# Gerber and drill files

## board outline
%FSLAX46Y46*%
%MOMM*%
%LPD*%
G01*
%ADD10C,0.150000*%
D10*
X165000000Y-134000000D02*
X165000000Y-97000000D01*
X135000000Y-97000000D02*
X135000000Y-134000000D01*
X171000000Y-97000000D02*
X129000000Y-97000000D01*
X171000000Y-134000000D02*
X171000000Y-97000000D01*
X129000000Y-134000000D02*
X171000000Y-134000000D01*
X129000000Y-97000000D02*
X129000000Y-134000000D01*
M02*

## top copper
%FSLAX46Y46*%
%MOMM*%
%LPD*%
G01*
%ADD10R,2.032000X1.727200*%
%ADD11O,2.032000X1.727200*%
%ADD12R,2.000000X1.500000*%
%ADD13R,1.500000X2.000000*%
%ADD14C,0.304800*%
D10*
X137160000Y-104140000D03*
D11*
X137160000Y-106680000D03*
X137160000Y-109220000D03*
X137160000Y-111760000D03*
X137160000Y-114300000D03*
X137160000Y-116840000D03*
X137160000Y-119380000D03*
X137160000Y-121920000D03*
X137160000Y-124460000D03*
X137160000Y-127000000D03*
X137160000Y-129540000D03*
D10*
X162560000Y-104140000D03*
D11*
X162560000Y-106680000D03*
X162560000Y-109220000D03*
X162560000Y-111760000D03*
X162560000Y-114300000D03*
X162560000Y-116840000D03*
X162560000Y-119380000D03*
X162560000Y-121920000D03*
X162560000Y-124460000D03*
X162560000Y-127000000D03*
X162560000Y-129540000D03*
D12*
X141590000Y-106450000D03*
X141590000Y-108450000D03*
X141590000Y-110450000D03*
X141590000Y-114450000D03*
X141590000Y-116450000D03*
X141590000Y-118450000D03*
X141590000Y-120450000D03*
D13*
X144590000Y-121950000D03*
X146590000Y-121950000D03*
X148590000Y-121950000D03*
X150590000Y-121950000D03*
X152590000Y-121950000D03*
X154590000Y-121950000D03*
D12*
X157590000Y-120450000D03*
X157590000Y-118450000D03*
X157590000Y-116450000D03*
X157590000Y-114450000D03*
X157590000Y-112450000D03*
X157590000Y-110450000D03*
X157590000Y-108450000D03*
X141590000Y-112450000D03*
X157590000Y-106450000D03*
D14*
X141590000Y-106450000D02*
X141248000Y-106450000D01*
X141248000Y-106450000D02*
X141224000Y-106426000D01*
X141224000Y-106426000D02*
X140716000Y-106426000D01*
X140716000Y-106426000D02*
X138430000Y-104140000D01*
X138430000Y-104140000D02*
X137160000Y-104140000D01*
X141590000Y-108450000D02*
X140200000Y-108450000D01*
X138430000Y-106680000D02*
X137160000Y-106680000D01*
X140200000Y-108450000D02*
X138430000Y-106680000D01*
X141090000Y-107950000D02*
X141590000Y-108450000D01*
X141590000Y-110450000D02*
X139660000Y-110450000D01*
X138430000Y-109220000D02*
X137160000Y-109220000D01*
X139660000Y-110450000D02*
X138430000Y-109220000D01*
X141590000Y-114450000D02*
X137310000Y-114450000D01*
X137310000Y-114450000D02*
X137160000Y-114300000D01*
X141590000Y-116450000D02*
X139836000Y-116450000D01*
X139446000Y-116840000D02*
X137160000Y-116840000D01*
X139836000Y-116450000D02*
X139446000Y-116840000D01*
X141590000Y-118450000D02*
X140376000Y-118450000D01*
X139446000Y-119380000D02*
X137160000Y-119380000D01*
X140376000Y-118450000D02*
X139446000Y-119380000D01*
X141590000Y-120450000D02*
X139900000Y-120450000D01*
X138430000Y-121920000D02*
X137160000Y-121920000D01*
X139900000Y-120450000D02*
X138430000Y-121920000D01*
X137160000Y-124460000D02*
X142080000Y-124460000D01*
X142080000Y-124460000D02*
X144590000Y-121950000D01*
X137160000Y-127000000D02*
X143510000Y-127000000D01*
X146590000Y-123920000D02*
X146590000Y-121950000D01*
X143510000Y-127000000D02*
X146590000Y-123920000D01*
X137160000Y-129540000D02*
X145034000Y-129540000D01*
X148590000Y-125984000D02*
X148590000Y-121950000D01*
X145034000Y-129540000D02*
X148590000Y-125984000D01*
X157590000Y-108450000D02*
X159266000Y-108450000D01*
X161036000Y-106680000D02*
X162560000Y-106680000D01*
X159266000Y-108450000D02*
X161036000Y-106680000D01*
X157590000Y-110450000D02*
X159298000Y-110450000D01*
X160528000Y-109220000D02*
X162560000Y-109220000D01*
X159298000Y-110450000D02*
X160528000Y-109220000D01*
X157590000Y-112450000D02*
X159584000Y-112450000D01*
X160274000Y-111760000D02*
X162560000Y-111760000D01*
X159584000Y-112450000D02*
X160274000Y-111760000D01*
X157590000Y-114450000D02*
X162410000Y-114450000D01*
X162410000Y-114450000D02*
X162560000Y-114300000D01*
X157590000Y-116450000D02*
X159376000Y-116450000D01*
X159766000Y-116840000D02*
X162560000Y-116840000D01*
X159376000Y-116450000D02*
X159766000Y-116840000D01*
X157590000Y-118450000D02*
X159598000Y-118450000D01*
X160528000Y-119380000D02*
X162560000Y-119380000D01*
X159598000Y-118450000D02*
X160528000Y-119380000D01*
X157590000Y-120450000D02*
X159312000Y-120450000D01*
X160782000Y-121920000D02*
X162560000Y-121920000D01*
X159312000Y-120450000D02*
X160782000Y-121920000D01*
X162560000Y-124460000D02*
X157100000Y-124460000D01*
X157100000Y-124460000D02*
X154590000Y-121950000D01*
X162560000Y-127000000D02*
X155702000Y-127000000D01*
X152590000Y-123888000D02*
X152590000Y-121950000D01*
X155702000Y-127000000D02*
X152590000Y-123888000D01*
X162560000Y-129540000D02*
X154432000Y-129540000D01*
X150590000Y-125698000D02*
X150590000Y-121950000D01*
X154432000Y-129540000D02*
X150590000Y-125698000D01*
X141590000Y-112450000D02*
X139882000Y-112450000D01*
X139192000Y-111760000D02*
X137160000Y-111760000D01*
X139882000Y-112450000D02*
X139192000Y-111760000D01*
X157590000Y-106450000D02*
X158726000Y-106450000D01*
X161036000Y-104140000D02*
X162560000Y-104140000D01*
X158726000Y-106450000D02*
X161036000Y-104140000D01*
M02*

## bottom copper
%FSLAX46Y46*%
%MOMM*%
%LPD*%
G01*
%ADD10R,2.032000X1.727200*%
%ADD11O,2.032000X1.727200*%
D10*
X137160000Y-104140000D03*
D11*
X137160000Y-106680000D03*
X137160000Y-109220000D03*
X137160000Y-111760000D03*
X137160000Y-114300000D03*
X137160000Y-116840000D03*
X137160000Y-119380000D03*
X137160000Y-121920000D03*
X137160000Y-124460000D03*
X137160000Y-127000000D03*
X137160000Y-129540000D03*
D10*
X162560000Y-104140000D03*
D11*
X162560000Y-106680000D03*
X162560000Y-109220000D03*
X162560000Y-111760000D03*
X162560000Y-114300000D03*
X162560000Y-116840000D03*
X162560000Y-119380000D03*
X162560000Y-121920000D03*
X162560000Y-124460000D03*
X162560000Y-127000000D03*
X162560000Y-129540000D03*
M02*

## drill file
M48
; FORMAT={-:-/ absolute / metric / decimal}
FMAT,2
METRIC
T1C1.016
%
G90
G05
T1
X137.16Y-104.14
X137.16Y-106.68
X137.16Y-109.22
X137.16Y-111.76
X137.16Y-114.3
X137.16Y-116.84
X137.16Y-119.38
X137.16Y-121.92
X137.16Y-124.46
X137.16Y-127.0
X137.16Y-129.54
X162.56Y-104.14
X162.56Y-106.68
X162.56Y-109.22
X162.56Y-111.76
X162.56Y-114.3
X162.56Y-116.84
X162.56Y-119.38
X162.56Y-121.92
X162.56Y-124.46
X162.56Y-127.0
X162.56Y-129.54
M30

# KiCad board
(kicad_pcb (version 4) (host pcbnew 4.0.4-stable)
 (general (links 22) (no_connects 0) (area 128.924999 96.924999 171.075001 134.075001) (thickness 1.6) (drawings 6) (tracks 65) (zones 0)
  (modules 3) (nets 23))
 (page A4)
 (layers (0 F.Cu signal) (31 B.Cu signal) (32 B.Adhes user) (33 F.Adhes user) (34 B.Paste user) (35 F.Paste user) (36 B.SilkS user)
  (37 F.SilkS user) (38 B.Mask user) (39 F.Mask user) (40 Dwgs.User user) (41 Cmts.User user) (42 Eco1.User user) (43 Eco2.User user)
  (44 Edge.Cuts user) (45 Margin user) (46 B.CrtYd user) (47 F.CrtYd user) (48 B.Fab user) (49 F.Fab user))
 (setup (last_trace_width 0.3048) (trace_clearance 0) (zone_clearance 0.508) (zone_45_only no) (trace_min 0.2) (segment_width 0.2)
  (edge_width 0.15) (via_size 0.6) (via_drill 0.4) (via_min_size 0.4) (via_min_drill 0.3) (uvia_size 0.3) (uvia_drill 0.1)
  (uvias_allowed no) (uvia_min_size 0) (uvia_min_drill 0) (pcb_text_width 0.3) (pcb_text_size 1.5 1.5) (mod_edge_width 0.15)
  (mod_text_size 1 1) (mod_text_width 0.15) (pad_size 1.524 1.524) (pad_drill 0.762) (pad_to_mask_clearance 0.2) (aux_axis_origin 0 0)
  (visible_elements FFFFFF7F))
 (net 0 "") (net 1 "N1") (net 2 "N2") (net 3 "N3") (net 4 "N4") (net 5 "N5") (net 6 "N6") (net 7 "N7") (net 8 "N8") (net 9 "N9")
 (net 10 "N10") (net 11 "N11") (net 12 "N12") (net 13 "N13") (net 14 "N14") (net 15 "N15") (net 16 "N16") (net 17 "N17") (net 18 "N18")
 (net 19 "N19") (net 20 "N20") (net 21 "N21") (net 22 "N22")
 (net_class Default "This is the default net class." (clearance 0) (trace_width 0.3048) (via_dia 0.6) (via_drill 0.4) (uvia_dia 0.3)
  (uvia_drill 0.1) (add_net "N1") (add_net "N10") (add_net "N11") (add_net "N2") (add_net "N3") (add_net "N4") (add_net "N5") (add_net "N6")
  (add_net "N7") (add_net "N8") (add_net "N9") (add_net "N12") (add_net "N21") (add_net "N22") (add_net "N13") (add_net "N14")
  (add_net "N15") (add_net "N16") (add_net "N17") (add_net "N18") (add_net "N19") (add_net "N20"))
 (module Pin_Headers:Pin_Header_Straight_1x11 (layer F.Cu) (at 137.16 104.14)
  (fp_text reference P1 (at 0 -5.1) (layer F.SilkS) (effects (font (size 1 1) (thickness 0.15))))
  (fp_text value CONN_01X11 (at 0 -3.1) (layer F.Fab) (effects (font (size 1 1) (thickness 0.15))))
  (pad 1 thru_hole rect (at 0 0) (size 2.032 1.7272) (drill 1.016) (layers *.Cu *.Mask F.SilkS) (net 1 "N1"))
  (pad 2 thru_hole oval (at 0 2.54) (size 2.032 1.7272) (drill 1.016) (layers *.Cu *.Mask F.SilkS) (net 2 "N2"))
  (pad 3 thru_hole oval (at 0 5.08) (size 2.032 1.7272) (drill 1.016) (layers *.Cu *.Mask F.SilkS) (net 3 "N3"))
  (pad 4 thru_hole oval (at 0 7.62) (size 2.032 1.7272) (drill 1.016) (layers *.Cu *.Mask F.SilkS) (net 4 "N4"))
  (pad 5 thru_hole oval (at 0 10.16) (size 2.032 1.7272) (drill 1.016) (layers *.Cu *.Mask F.SilkS) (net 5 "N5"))
  (pad 6 thru_hole oval (at 0 12.7) (size 2.032 1.7272) (drill 1.016) (layers *.Cu *.Mask F.SilkS) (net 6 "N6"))
  (pad 7 thru_hole oval (at 0 15.24) (size 2.032 1.7272) (drill 1.016) (layers *.Cu *.Mask F.SilkS) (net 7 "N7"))
  (pad 8 thru_hole oval (at 0 17.78) (size 2.032 1.7272) (drill 1.016) (layers *.Cu *.Mask F.SilkS) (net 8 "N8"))
  (pad 9 thru_hole oval (at 0 20.32) (size 2.032 1.7272) (drill 1.016) (layers *.Cu *.Mask F.SilkS) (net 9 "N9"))
  (pad 10 thru_hole oval (at 0 22.86) (size 2.032 1.7272) (drill 1.016) (layers *.Cu *.Mask F.SilkS) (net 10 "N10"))
  (pad 11 thru_hole oval (at 0 25.4) (size 2.032 1.7272) (drill 1.016) (layers *.Cu *.Mask F.SilkS) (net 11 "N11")))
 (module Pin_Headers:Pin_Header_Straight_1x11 (layer F.Cu) (at 162.56 104.14)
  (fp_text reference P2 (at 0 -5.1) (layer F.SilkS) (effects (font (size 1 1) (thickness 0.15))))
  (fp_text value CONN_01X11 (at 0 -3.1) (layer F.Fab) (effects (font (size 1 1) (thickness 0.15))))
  (pad 1 thru_hole rect (at 0 0) (size 2.032 1.7272) (drill 1.016) (layers *.Cu *.Mask F.SilkS) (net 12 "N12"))
  (pad 2 thru_hole oval (at 0 2.54) (size 2.032 1.7272) (drill 1.016) (layers *.Cu *.Mask F.SilkS) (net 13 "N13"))
  (pad 3 thru_hole oval (at 0 5.08) (size 2.032 1.7272) (drill 1.016) (layers *.Cu *.Mask F.SilkS) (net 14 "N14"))
  (pad 4 thru_hole oval (at 0 7.62) (size 2.032 1.7272) (drill 1.016) (layers *.Cu *.Mask F.SilkS) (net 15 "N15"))
  (pad 5 thru_hole oval (at 0 10.16) (size 2.032 1.7272) (drill 1.016) (layers *.Cu *.Mask F.SilkS) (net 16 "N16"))
  (pad 6 thru_hole oval (at 0 12.7) (size 2.032 1.7272) (drill 1.016) (layers *.Cu *.Mask F.SilkS) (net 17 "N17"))
  (pad 7 thru_hole oval (at 0 15.24) (size 2.032 1.7272) (drill 1.016) (layers *.Cu *.Mask F.SilkS) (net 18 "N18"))
  (pad 8 thru_hole oval (at 0 17.78) (size 2.032 1.7272) (drill 1.016) (layers *.Cu *.Mask F.SilkS) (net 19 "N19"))
  (pad 9 thru_hole oval (at 0 20.32) (size 2.032 1.7272) (drill 1.016) (layers *.Cu *.Mask F.SilkS) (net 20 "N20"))
  (pad 10 thru_hole oval (at 0 22.86) (size 2.032 1.7272) (drill 1.016) (layers *.Cu *.Mask F.SilkS) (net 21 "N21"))
  (pad 11 thru_hole oval (at 0 25.4) (size 2.032 1.7272) (drill 1.016) (layers *.Cu *.Mask F.SilkS) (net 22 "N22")))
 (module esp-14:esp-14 (layer F.Cu) (at 148.59 107.95)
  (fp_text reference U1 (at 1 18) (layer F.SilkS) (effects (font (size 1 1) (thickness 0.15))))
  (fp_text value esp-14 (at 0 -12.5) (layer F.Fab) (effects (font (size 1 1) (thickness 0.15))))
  (pad 1 smd rect (at -7 -1.5) (size 2 1.5) (layers F.Cu F.Paste F.Mask) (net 1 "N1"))
  (pad 2 smd rect (at -7 0.5) (size 2 1.5) (layers F.Cu F.Paste F.Mask) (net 2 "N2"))
  (pad 3 smd rect (at -7 2.5) (size 2 1.5) (layers F.Cu F.Paste F.Mask) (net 3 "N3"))
  (pad 5 smd rect (at -7 6.5) (size 2 1.5) (layers F.Cu F.Paste F.Mask) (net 5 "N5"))
  (pad 6 smd rect (at -7 8.5) (size 2 1.5) (layers F.Cu F.Paste F.Mask) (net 6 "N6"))
  (pad 7 smd rect (at -7 10.5) (size 2 1.5) (layers F.Cu F.Paste F.Mask) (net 7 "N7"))
  (pad 8 smd rect (at -7 12.5) (size 2 1.5) (layers F.Cu F.Paste F.Mask) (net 8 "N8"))
  (pad 9 smd rect (at -4 14) (size 1.5 2) (layers F.Cu F.Paste F.Mask) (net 9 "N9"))
  (pad 10 smd rect (at -2 14) (size 1.5 2) (layers F.Cu F.Paste F.Mask) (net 10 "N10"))
  (pad 11 smd rect (at 0 14) (size 1.5 2) (layers F.Cu F.Paste F.Mask) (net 11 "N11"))
  (pad 12 smd rect (at 2 14) (size 1.5 2) (layers F.Cu F.Paste F.Mask) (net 22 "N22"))
  (pad 13 smd rect (at 4 14) (size 1.5 2) (layers F.Cu F.Paste F.Mask) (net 21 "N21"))
  (pad 14 smd rect (at 6 14) (size 1.5 2) (layers F.Cu F.Paste F.Mask) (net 20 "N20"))
  (pad 15 smd rect (at 9 12.5) (size 2 1.5) (layers F.Cu F.Paste F.Mask) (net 19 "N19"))
  (pad 16 smd rect (at 9 10.5) (size 2 1.5) (layers F.Cu F.Paste F.Mask) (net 18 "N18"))
  (pad 17 smd rect (at 9 8.5) (size 2 1.5) (layers F.Cu F.Paste F.Mask) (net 17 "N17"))
  (pad 18 smd rect (at 9 6.5) (size 2 1.5) (layers F.Cu F.Paste F.Mask) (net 16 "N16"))
  (pad 19 smd rect (at 9 4.5) (size 2 1.5) (layers F.Cu F.Paste F.Mask) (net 15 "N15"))
  (pad 20 smd rect (at 9 2.5) (size 2 1.5) (layers F.Cu F.Paste F.Mask) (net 14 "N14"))
  (pad 21 smd rect (at 9 0.5) (size 2 1.5) (layers F.Cu F.Paste F.Mask) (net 13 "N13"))
  (pad 4 smd rect (at -7 4.5) (size 2 1.5) (layers F.Cu F.Paste F.Mask) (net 4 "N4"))
  (pad 22 smd rect (at 9 -1.5) (size 2 1.5) (layers F.Cu F.Paste F.Mask) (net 12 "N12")))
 (gr_line (start 165 134) (end 165 97) (angle 90) (layer Edge.Cuts) (width 0.15))
 (gr_line (start 135 97) (end 135 134) (angle 90) (layer Edge.Cuts) (width 0.15))
 (gr_line (start 171 97) (end 129 97) (angle 90) (layer Edge.Cuts) (width 0.15))
 (gr_line (start 171 134) (end 171 97) (angle 90) (layer Edge.Cuts) (width 0.15))
 (gr_line (start 129 134) (end 171 134) (angle 90) (layer Edge.Cuts) (width 0.15))
 (gr_line (start 129 97) (end 129 134) (angle 90) (layer Edge.Cuts) (width 0.15))
 (segment (start 141.59 106.45) (end 141.248 106.45) (width 0.3048) (layer F.Cu) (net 1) (status C00000))
 (segment (start 141.248 106.45) (end 141.224 106.426) (width 0.3048) (layer F.Cu) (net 1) (status C00000))
 (segment (start 141.224 106.426) (end 140.716 106.426) (width 0.3048) (layer F.Cu) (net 1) (status C00000))
 (segment (start 140.716 106.426) (end 138.43 104.14) (width 0.3048) (layer F.Cu) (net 1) (status 400000))
 (segment (start 138.43 104.14) (end 137.16 104.14) (width 0.3048) (layer F.Cu) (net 1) (status 800000))
 (segment (start 141.59 108.45) (end 140.2 108.45) (width 0.3048) (layer F.Cu) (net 2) (status 400000))
 (segment (start 138.43 106.68) (end 137.16 106.68) (width 0.3048) (layer F.Cu) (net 2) (status 800000))
 (segment (start 140.2 108.45) (end 138.43 106.68) (width 0.3048) (layer F.Cu) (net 2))
 (segment (start 141.09 107.95) (end 141.59 108.45) (width 0.3048) (layer F.Cu) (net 2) (status C00000))
 (segment (start 141.59 110.45) (end 139.66 110.45) (width 0.3048) (layer F.Cu) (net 3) (status 400000))
 (segment (start 138.43 109.22) (end 137.16 109.22) (width 0.3048) (layer F.Cu) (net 3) (status 800000))
 (segment (start 139.66 110.45) (end 138.43 109.22) (width 0.3048) (layer F.Cu) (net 3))
 (segment (start 141.59 114.45) (end 137.31 114.45) (width 0.3048) (layer F.Cu) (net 5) (status C00000))
 (segment (start 137.31 114.45) (end 137.16 114.3) (width 0.3048) (layer F.Cu) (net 5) (status C00000))
 (segment (start 141.59 116.45) (end 139.836 116.45) (width 0.3048) (layer F.Cu) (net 6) (status 400000))
 (segment (start 139.446 116.84) (end 137.16 116.84) (width 0.3048) (layer F.Cu) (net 6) (status 800000))
 (segment (start 139.836 116.45) (end 139.446 116.84) (width 0.3048) (layer F.Cu) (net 6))
 (segment (start 141.59 118.45) (end 140.376 118.45) (width 0.3048) (layer F.Cu) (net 7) (status 400000))
 (segment (start 139.446 119.38) (end 137.16 119.38) (width 0.3048) (layer F.Cu) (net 7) (status 800000))
 (segment (start 140.376 118.45) (end 139.446 119.38) (width 0.3048) (layer F.Cu) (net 7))
 (segment (start 141.59 120.45) (end 139.9 120.45) (width 0.3048) (layer F.Cu) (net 8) (status 400000))
 (segment (start 138.43 121.92) (end 137.16 121.92) (width 0.3048) (layer F.Cu) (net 8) (status 800000))
 (segment (start 139.9 120.45) (end 138.43 121.92) (width 0.3048) (layer F.Cu) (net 8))
 (segment (start 137.16 124.46) (end 142.08 124.46) (width 0.3048) (layer F.Cu) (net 9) (status 400000))
 (segment (start 142.08 124.46) (end 144.59 121.95) (width 0.3048) (layer F.Cu) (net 9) (status 800000))
 (segment (start 137.16 127) (end 143.51 127) (width 0.3048) (layer F.Cu) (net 10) (status 400000))
 (segment (start 146.59 123.92) (end 146.59 121.95) (width 0.3048) (layer F.Cu) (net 10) (status 800000))
 (segment (start 143.51 127) (end 146.59 123.92) (width 0.3048) (layer F.Cu) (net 10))
 (segment (start 137.16 129.54) (end 145.034 129.54) (width 0.3048) (layer F.Cu) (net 11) (status 400000))
 (segment (start 148.59 125.984) (end 148.59 121.95) (width 0.3048) (layer F.Cu) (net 11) (status 800000))
 (segment (start 145.034 129.54) (end 148.59 125.984) (width 0.3048) (layer F.Cu) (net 11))
 (segment (start 157.59 108.45) (end 159.266 108.45) (width 0.3048) (layer F.Cu) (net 13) (status 400000))
 (segment (start 161.036 106.68) (end 162.56 106.68) (width 0.3048) (layer F.Cu) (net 13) (status 800000))
 (segment (start 159.266 108.45) (end 161.036 106.68) (width 0.3048) (layer F.Cu) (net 13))
 (segment (start 157.59 110.45) (end 159.298 110.45) (width 0.3048) (layer F.Cu) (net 14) (status 400000))
 (segment (start 160.528 109.22) (end 162.56 109.22) (width 0.3048) (layer F.Cu) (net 14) (status 800000))
 (segment (start 159.298 110.45) (end 160.528 109.22) (width 0.3048) (layer F.Cu) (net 14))
 (segment (start 157.59 112.45) (end 159.584 112.45) (width 0.3048) (layer F.Cu) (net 15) (status 400000))
 (segment (start 160.274 111.76) (end 162.56 111.76) (width 0.3048) (layer F.Cu) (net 15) (status 800000))
 (segment (start 159.584 112.45) (end 160.274 111.76) (width 0.3048) (layer F.Cu) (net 15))
 (segment (start 157.59 114.45) (end 162.41 114.45) (width 0.3048) (layer F.Cu) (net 16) (status C00000))
 (segment (start 162.41 114.45) (end 162.56 114.3) (width 0.3048) (layer F.Cu) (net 16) (status C00000))
 (segment (start 157.59 116.45) (end 159.376 116.45) (width 0.3048) (layer F.Cu) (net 17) (status 400000))
 (segment (start 159.766 116.84) (end 162.56 116.84) (width 0.3048) (layer F.Cu) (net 17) (status 800000))
 (segment (start 159.376 116.45) (end 159.766 116.84) (width 0.3048) (layer F.Cu) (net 17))
 (segment (start 157.59 118.45) (end 159.598 118.45) (width 0.3048) (layer F.Cu) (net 18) (status 400000))
 (segment (start 160.528 119.38) (end 162.56 119.38) (width 0.3048) (layer F.Cu) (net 18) (status 800000))
 (segment (start 159.598 118.45) (end 160.528 119.38) (width 0.3048) (layer F.Cu) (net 18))
 (segment (start 157.59 120.45) (end 159.312 120.45) (width 0.3048) (layer F.Cu) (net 19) (status 400000))
 (segment (start 160.782 121.92) (end 162.56 121.92) (width 0.3048) (layer F.Cu) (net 19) (status 800000))
 (segment (start 159.312 120.45) (end 160.782 121.92) (width 0.3048) (layer F.Cu) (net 19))
 (segment (start 162.56 124.46) (end 157.1 124.46) (width 0.3048) (layer F.Cu) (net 20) (status 400000))
 (segment (start 157.1 124.46) (end 154.59 121.95) (width 0.3048) (layer F.Cu) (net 20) (status 800000))
 (segment (start 162.56 127) (end 155.702 127) (width 0.3048) (layer F.Cu) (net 21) (status 400000))
 (segment (start 152.59 123.888) (end 152.59 121.95) (width 0.3048) (layer F.Cu) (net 21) (status 800000))
 (segment (start 155.702 127) (end 152.59 123.888) (width 0.3048) (layer F.Cu) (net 21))
 (segment (start 162.56 129.54) (end 154.432 129.54) (width 0.3048) (layer F.Cu) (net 22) (status 400000))
 (segment (start 150.59 125.698) (end 150.59 121.95) (width 0.3048) (layer F.Cu) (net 22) (status 800000))
 (segment (start 154.432 129.54) (end 150.59 125.698) (width 0.3048) (layer F.Cu) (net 22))
 (segment (start 141.59 112.45) (end 139.882 112.45) (width 0.3048) (layer F.Cu) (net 4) (status 400000))
 (segment (start 139.192 111.76) (end 137.16 111.76) (width 0.3048) (layer F.Cu) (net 4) (status 800000))
 (segment (start 139.882 112.45) (end 139.192 111.76) (width 0.3048) (layer F.Cu) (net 4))
 (segment (start 157.59 106.45) (end 158.726 106.45) (width 0.3048) (layer F.Cu) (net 12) (status 400000))
 (segment (start 161.036 104.14) (end 162.56 104.14) (width 0.3048) (layer F.Cu) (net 12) (status 800000))
 (segment (start 158.726 106.45) (end 161.036 104.14) (width 0.3048) (layer F.Cu) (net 12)))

